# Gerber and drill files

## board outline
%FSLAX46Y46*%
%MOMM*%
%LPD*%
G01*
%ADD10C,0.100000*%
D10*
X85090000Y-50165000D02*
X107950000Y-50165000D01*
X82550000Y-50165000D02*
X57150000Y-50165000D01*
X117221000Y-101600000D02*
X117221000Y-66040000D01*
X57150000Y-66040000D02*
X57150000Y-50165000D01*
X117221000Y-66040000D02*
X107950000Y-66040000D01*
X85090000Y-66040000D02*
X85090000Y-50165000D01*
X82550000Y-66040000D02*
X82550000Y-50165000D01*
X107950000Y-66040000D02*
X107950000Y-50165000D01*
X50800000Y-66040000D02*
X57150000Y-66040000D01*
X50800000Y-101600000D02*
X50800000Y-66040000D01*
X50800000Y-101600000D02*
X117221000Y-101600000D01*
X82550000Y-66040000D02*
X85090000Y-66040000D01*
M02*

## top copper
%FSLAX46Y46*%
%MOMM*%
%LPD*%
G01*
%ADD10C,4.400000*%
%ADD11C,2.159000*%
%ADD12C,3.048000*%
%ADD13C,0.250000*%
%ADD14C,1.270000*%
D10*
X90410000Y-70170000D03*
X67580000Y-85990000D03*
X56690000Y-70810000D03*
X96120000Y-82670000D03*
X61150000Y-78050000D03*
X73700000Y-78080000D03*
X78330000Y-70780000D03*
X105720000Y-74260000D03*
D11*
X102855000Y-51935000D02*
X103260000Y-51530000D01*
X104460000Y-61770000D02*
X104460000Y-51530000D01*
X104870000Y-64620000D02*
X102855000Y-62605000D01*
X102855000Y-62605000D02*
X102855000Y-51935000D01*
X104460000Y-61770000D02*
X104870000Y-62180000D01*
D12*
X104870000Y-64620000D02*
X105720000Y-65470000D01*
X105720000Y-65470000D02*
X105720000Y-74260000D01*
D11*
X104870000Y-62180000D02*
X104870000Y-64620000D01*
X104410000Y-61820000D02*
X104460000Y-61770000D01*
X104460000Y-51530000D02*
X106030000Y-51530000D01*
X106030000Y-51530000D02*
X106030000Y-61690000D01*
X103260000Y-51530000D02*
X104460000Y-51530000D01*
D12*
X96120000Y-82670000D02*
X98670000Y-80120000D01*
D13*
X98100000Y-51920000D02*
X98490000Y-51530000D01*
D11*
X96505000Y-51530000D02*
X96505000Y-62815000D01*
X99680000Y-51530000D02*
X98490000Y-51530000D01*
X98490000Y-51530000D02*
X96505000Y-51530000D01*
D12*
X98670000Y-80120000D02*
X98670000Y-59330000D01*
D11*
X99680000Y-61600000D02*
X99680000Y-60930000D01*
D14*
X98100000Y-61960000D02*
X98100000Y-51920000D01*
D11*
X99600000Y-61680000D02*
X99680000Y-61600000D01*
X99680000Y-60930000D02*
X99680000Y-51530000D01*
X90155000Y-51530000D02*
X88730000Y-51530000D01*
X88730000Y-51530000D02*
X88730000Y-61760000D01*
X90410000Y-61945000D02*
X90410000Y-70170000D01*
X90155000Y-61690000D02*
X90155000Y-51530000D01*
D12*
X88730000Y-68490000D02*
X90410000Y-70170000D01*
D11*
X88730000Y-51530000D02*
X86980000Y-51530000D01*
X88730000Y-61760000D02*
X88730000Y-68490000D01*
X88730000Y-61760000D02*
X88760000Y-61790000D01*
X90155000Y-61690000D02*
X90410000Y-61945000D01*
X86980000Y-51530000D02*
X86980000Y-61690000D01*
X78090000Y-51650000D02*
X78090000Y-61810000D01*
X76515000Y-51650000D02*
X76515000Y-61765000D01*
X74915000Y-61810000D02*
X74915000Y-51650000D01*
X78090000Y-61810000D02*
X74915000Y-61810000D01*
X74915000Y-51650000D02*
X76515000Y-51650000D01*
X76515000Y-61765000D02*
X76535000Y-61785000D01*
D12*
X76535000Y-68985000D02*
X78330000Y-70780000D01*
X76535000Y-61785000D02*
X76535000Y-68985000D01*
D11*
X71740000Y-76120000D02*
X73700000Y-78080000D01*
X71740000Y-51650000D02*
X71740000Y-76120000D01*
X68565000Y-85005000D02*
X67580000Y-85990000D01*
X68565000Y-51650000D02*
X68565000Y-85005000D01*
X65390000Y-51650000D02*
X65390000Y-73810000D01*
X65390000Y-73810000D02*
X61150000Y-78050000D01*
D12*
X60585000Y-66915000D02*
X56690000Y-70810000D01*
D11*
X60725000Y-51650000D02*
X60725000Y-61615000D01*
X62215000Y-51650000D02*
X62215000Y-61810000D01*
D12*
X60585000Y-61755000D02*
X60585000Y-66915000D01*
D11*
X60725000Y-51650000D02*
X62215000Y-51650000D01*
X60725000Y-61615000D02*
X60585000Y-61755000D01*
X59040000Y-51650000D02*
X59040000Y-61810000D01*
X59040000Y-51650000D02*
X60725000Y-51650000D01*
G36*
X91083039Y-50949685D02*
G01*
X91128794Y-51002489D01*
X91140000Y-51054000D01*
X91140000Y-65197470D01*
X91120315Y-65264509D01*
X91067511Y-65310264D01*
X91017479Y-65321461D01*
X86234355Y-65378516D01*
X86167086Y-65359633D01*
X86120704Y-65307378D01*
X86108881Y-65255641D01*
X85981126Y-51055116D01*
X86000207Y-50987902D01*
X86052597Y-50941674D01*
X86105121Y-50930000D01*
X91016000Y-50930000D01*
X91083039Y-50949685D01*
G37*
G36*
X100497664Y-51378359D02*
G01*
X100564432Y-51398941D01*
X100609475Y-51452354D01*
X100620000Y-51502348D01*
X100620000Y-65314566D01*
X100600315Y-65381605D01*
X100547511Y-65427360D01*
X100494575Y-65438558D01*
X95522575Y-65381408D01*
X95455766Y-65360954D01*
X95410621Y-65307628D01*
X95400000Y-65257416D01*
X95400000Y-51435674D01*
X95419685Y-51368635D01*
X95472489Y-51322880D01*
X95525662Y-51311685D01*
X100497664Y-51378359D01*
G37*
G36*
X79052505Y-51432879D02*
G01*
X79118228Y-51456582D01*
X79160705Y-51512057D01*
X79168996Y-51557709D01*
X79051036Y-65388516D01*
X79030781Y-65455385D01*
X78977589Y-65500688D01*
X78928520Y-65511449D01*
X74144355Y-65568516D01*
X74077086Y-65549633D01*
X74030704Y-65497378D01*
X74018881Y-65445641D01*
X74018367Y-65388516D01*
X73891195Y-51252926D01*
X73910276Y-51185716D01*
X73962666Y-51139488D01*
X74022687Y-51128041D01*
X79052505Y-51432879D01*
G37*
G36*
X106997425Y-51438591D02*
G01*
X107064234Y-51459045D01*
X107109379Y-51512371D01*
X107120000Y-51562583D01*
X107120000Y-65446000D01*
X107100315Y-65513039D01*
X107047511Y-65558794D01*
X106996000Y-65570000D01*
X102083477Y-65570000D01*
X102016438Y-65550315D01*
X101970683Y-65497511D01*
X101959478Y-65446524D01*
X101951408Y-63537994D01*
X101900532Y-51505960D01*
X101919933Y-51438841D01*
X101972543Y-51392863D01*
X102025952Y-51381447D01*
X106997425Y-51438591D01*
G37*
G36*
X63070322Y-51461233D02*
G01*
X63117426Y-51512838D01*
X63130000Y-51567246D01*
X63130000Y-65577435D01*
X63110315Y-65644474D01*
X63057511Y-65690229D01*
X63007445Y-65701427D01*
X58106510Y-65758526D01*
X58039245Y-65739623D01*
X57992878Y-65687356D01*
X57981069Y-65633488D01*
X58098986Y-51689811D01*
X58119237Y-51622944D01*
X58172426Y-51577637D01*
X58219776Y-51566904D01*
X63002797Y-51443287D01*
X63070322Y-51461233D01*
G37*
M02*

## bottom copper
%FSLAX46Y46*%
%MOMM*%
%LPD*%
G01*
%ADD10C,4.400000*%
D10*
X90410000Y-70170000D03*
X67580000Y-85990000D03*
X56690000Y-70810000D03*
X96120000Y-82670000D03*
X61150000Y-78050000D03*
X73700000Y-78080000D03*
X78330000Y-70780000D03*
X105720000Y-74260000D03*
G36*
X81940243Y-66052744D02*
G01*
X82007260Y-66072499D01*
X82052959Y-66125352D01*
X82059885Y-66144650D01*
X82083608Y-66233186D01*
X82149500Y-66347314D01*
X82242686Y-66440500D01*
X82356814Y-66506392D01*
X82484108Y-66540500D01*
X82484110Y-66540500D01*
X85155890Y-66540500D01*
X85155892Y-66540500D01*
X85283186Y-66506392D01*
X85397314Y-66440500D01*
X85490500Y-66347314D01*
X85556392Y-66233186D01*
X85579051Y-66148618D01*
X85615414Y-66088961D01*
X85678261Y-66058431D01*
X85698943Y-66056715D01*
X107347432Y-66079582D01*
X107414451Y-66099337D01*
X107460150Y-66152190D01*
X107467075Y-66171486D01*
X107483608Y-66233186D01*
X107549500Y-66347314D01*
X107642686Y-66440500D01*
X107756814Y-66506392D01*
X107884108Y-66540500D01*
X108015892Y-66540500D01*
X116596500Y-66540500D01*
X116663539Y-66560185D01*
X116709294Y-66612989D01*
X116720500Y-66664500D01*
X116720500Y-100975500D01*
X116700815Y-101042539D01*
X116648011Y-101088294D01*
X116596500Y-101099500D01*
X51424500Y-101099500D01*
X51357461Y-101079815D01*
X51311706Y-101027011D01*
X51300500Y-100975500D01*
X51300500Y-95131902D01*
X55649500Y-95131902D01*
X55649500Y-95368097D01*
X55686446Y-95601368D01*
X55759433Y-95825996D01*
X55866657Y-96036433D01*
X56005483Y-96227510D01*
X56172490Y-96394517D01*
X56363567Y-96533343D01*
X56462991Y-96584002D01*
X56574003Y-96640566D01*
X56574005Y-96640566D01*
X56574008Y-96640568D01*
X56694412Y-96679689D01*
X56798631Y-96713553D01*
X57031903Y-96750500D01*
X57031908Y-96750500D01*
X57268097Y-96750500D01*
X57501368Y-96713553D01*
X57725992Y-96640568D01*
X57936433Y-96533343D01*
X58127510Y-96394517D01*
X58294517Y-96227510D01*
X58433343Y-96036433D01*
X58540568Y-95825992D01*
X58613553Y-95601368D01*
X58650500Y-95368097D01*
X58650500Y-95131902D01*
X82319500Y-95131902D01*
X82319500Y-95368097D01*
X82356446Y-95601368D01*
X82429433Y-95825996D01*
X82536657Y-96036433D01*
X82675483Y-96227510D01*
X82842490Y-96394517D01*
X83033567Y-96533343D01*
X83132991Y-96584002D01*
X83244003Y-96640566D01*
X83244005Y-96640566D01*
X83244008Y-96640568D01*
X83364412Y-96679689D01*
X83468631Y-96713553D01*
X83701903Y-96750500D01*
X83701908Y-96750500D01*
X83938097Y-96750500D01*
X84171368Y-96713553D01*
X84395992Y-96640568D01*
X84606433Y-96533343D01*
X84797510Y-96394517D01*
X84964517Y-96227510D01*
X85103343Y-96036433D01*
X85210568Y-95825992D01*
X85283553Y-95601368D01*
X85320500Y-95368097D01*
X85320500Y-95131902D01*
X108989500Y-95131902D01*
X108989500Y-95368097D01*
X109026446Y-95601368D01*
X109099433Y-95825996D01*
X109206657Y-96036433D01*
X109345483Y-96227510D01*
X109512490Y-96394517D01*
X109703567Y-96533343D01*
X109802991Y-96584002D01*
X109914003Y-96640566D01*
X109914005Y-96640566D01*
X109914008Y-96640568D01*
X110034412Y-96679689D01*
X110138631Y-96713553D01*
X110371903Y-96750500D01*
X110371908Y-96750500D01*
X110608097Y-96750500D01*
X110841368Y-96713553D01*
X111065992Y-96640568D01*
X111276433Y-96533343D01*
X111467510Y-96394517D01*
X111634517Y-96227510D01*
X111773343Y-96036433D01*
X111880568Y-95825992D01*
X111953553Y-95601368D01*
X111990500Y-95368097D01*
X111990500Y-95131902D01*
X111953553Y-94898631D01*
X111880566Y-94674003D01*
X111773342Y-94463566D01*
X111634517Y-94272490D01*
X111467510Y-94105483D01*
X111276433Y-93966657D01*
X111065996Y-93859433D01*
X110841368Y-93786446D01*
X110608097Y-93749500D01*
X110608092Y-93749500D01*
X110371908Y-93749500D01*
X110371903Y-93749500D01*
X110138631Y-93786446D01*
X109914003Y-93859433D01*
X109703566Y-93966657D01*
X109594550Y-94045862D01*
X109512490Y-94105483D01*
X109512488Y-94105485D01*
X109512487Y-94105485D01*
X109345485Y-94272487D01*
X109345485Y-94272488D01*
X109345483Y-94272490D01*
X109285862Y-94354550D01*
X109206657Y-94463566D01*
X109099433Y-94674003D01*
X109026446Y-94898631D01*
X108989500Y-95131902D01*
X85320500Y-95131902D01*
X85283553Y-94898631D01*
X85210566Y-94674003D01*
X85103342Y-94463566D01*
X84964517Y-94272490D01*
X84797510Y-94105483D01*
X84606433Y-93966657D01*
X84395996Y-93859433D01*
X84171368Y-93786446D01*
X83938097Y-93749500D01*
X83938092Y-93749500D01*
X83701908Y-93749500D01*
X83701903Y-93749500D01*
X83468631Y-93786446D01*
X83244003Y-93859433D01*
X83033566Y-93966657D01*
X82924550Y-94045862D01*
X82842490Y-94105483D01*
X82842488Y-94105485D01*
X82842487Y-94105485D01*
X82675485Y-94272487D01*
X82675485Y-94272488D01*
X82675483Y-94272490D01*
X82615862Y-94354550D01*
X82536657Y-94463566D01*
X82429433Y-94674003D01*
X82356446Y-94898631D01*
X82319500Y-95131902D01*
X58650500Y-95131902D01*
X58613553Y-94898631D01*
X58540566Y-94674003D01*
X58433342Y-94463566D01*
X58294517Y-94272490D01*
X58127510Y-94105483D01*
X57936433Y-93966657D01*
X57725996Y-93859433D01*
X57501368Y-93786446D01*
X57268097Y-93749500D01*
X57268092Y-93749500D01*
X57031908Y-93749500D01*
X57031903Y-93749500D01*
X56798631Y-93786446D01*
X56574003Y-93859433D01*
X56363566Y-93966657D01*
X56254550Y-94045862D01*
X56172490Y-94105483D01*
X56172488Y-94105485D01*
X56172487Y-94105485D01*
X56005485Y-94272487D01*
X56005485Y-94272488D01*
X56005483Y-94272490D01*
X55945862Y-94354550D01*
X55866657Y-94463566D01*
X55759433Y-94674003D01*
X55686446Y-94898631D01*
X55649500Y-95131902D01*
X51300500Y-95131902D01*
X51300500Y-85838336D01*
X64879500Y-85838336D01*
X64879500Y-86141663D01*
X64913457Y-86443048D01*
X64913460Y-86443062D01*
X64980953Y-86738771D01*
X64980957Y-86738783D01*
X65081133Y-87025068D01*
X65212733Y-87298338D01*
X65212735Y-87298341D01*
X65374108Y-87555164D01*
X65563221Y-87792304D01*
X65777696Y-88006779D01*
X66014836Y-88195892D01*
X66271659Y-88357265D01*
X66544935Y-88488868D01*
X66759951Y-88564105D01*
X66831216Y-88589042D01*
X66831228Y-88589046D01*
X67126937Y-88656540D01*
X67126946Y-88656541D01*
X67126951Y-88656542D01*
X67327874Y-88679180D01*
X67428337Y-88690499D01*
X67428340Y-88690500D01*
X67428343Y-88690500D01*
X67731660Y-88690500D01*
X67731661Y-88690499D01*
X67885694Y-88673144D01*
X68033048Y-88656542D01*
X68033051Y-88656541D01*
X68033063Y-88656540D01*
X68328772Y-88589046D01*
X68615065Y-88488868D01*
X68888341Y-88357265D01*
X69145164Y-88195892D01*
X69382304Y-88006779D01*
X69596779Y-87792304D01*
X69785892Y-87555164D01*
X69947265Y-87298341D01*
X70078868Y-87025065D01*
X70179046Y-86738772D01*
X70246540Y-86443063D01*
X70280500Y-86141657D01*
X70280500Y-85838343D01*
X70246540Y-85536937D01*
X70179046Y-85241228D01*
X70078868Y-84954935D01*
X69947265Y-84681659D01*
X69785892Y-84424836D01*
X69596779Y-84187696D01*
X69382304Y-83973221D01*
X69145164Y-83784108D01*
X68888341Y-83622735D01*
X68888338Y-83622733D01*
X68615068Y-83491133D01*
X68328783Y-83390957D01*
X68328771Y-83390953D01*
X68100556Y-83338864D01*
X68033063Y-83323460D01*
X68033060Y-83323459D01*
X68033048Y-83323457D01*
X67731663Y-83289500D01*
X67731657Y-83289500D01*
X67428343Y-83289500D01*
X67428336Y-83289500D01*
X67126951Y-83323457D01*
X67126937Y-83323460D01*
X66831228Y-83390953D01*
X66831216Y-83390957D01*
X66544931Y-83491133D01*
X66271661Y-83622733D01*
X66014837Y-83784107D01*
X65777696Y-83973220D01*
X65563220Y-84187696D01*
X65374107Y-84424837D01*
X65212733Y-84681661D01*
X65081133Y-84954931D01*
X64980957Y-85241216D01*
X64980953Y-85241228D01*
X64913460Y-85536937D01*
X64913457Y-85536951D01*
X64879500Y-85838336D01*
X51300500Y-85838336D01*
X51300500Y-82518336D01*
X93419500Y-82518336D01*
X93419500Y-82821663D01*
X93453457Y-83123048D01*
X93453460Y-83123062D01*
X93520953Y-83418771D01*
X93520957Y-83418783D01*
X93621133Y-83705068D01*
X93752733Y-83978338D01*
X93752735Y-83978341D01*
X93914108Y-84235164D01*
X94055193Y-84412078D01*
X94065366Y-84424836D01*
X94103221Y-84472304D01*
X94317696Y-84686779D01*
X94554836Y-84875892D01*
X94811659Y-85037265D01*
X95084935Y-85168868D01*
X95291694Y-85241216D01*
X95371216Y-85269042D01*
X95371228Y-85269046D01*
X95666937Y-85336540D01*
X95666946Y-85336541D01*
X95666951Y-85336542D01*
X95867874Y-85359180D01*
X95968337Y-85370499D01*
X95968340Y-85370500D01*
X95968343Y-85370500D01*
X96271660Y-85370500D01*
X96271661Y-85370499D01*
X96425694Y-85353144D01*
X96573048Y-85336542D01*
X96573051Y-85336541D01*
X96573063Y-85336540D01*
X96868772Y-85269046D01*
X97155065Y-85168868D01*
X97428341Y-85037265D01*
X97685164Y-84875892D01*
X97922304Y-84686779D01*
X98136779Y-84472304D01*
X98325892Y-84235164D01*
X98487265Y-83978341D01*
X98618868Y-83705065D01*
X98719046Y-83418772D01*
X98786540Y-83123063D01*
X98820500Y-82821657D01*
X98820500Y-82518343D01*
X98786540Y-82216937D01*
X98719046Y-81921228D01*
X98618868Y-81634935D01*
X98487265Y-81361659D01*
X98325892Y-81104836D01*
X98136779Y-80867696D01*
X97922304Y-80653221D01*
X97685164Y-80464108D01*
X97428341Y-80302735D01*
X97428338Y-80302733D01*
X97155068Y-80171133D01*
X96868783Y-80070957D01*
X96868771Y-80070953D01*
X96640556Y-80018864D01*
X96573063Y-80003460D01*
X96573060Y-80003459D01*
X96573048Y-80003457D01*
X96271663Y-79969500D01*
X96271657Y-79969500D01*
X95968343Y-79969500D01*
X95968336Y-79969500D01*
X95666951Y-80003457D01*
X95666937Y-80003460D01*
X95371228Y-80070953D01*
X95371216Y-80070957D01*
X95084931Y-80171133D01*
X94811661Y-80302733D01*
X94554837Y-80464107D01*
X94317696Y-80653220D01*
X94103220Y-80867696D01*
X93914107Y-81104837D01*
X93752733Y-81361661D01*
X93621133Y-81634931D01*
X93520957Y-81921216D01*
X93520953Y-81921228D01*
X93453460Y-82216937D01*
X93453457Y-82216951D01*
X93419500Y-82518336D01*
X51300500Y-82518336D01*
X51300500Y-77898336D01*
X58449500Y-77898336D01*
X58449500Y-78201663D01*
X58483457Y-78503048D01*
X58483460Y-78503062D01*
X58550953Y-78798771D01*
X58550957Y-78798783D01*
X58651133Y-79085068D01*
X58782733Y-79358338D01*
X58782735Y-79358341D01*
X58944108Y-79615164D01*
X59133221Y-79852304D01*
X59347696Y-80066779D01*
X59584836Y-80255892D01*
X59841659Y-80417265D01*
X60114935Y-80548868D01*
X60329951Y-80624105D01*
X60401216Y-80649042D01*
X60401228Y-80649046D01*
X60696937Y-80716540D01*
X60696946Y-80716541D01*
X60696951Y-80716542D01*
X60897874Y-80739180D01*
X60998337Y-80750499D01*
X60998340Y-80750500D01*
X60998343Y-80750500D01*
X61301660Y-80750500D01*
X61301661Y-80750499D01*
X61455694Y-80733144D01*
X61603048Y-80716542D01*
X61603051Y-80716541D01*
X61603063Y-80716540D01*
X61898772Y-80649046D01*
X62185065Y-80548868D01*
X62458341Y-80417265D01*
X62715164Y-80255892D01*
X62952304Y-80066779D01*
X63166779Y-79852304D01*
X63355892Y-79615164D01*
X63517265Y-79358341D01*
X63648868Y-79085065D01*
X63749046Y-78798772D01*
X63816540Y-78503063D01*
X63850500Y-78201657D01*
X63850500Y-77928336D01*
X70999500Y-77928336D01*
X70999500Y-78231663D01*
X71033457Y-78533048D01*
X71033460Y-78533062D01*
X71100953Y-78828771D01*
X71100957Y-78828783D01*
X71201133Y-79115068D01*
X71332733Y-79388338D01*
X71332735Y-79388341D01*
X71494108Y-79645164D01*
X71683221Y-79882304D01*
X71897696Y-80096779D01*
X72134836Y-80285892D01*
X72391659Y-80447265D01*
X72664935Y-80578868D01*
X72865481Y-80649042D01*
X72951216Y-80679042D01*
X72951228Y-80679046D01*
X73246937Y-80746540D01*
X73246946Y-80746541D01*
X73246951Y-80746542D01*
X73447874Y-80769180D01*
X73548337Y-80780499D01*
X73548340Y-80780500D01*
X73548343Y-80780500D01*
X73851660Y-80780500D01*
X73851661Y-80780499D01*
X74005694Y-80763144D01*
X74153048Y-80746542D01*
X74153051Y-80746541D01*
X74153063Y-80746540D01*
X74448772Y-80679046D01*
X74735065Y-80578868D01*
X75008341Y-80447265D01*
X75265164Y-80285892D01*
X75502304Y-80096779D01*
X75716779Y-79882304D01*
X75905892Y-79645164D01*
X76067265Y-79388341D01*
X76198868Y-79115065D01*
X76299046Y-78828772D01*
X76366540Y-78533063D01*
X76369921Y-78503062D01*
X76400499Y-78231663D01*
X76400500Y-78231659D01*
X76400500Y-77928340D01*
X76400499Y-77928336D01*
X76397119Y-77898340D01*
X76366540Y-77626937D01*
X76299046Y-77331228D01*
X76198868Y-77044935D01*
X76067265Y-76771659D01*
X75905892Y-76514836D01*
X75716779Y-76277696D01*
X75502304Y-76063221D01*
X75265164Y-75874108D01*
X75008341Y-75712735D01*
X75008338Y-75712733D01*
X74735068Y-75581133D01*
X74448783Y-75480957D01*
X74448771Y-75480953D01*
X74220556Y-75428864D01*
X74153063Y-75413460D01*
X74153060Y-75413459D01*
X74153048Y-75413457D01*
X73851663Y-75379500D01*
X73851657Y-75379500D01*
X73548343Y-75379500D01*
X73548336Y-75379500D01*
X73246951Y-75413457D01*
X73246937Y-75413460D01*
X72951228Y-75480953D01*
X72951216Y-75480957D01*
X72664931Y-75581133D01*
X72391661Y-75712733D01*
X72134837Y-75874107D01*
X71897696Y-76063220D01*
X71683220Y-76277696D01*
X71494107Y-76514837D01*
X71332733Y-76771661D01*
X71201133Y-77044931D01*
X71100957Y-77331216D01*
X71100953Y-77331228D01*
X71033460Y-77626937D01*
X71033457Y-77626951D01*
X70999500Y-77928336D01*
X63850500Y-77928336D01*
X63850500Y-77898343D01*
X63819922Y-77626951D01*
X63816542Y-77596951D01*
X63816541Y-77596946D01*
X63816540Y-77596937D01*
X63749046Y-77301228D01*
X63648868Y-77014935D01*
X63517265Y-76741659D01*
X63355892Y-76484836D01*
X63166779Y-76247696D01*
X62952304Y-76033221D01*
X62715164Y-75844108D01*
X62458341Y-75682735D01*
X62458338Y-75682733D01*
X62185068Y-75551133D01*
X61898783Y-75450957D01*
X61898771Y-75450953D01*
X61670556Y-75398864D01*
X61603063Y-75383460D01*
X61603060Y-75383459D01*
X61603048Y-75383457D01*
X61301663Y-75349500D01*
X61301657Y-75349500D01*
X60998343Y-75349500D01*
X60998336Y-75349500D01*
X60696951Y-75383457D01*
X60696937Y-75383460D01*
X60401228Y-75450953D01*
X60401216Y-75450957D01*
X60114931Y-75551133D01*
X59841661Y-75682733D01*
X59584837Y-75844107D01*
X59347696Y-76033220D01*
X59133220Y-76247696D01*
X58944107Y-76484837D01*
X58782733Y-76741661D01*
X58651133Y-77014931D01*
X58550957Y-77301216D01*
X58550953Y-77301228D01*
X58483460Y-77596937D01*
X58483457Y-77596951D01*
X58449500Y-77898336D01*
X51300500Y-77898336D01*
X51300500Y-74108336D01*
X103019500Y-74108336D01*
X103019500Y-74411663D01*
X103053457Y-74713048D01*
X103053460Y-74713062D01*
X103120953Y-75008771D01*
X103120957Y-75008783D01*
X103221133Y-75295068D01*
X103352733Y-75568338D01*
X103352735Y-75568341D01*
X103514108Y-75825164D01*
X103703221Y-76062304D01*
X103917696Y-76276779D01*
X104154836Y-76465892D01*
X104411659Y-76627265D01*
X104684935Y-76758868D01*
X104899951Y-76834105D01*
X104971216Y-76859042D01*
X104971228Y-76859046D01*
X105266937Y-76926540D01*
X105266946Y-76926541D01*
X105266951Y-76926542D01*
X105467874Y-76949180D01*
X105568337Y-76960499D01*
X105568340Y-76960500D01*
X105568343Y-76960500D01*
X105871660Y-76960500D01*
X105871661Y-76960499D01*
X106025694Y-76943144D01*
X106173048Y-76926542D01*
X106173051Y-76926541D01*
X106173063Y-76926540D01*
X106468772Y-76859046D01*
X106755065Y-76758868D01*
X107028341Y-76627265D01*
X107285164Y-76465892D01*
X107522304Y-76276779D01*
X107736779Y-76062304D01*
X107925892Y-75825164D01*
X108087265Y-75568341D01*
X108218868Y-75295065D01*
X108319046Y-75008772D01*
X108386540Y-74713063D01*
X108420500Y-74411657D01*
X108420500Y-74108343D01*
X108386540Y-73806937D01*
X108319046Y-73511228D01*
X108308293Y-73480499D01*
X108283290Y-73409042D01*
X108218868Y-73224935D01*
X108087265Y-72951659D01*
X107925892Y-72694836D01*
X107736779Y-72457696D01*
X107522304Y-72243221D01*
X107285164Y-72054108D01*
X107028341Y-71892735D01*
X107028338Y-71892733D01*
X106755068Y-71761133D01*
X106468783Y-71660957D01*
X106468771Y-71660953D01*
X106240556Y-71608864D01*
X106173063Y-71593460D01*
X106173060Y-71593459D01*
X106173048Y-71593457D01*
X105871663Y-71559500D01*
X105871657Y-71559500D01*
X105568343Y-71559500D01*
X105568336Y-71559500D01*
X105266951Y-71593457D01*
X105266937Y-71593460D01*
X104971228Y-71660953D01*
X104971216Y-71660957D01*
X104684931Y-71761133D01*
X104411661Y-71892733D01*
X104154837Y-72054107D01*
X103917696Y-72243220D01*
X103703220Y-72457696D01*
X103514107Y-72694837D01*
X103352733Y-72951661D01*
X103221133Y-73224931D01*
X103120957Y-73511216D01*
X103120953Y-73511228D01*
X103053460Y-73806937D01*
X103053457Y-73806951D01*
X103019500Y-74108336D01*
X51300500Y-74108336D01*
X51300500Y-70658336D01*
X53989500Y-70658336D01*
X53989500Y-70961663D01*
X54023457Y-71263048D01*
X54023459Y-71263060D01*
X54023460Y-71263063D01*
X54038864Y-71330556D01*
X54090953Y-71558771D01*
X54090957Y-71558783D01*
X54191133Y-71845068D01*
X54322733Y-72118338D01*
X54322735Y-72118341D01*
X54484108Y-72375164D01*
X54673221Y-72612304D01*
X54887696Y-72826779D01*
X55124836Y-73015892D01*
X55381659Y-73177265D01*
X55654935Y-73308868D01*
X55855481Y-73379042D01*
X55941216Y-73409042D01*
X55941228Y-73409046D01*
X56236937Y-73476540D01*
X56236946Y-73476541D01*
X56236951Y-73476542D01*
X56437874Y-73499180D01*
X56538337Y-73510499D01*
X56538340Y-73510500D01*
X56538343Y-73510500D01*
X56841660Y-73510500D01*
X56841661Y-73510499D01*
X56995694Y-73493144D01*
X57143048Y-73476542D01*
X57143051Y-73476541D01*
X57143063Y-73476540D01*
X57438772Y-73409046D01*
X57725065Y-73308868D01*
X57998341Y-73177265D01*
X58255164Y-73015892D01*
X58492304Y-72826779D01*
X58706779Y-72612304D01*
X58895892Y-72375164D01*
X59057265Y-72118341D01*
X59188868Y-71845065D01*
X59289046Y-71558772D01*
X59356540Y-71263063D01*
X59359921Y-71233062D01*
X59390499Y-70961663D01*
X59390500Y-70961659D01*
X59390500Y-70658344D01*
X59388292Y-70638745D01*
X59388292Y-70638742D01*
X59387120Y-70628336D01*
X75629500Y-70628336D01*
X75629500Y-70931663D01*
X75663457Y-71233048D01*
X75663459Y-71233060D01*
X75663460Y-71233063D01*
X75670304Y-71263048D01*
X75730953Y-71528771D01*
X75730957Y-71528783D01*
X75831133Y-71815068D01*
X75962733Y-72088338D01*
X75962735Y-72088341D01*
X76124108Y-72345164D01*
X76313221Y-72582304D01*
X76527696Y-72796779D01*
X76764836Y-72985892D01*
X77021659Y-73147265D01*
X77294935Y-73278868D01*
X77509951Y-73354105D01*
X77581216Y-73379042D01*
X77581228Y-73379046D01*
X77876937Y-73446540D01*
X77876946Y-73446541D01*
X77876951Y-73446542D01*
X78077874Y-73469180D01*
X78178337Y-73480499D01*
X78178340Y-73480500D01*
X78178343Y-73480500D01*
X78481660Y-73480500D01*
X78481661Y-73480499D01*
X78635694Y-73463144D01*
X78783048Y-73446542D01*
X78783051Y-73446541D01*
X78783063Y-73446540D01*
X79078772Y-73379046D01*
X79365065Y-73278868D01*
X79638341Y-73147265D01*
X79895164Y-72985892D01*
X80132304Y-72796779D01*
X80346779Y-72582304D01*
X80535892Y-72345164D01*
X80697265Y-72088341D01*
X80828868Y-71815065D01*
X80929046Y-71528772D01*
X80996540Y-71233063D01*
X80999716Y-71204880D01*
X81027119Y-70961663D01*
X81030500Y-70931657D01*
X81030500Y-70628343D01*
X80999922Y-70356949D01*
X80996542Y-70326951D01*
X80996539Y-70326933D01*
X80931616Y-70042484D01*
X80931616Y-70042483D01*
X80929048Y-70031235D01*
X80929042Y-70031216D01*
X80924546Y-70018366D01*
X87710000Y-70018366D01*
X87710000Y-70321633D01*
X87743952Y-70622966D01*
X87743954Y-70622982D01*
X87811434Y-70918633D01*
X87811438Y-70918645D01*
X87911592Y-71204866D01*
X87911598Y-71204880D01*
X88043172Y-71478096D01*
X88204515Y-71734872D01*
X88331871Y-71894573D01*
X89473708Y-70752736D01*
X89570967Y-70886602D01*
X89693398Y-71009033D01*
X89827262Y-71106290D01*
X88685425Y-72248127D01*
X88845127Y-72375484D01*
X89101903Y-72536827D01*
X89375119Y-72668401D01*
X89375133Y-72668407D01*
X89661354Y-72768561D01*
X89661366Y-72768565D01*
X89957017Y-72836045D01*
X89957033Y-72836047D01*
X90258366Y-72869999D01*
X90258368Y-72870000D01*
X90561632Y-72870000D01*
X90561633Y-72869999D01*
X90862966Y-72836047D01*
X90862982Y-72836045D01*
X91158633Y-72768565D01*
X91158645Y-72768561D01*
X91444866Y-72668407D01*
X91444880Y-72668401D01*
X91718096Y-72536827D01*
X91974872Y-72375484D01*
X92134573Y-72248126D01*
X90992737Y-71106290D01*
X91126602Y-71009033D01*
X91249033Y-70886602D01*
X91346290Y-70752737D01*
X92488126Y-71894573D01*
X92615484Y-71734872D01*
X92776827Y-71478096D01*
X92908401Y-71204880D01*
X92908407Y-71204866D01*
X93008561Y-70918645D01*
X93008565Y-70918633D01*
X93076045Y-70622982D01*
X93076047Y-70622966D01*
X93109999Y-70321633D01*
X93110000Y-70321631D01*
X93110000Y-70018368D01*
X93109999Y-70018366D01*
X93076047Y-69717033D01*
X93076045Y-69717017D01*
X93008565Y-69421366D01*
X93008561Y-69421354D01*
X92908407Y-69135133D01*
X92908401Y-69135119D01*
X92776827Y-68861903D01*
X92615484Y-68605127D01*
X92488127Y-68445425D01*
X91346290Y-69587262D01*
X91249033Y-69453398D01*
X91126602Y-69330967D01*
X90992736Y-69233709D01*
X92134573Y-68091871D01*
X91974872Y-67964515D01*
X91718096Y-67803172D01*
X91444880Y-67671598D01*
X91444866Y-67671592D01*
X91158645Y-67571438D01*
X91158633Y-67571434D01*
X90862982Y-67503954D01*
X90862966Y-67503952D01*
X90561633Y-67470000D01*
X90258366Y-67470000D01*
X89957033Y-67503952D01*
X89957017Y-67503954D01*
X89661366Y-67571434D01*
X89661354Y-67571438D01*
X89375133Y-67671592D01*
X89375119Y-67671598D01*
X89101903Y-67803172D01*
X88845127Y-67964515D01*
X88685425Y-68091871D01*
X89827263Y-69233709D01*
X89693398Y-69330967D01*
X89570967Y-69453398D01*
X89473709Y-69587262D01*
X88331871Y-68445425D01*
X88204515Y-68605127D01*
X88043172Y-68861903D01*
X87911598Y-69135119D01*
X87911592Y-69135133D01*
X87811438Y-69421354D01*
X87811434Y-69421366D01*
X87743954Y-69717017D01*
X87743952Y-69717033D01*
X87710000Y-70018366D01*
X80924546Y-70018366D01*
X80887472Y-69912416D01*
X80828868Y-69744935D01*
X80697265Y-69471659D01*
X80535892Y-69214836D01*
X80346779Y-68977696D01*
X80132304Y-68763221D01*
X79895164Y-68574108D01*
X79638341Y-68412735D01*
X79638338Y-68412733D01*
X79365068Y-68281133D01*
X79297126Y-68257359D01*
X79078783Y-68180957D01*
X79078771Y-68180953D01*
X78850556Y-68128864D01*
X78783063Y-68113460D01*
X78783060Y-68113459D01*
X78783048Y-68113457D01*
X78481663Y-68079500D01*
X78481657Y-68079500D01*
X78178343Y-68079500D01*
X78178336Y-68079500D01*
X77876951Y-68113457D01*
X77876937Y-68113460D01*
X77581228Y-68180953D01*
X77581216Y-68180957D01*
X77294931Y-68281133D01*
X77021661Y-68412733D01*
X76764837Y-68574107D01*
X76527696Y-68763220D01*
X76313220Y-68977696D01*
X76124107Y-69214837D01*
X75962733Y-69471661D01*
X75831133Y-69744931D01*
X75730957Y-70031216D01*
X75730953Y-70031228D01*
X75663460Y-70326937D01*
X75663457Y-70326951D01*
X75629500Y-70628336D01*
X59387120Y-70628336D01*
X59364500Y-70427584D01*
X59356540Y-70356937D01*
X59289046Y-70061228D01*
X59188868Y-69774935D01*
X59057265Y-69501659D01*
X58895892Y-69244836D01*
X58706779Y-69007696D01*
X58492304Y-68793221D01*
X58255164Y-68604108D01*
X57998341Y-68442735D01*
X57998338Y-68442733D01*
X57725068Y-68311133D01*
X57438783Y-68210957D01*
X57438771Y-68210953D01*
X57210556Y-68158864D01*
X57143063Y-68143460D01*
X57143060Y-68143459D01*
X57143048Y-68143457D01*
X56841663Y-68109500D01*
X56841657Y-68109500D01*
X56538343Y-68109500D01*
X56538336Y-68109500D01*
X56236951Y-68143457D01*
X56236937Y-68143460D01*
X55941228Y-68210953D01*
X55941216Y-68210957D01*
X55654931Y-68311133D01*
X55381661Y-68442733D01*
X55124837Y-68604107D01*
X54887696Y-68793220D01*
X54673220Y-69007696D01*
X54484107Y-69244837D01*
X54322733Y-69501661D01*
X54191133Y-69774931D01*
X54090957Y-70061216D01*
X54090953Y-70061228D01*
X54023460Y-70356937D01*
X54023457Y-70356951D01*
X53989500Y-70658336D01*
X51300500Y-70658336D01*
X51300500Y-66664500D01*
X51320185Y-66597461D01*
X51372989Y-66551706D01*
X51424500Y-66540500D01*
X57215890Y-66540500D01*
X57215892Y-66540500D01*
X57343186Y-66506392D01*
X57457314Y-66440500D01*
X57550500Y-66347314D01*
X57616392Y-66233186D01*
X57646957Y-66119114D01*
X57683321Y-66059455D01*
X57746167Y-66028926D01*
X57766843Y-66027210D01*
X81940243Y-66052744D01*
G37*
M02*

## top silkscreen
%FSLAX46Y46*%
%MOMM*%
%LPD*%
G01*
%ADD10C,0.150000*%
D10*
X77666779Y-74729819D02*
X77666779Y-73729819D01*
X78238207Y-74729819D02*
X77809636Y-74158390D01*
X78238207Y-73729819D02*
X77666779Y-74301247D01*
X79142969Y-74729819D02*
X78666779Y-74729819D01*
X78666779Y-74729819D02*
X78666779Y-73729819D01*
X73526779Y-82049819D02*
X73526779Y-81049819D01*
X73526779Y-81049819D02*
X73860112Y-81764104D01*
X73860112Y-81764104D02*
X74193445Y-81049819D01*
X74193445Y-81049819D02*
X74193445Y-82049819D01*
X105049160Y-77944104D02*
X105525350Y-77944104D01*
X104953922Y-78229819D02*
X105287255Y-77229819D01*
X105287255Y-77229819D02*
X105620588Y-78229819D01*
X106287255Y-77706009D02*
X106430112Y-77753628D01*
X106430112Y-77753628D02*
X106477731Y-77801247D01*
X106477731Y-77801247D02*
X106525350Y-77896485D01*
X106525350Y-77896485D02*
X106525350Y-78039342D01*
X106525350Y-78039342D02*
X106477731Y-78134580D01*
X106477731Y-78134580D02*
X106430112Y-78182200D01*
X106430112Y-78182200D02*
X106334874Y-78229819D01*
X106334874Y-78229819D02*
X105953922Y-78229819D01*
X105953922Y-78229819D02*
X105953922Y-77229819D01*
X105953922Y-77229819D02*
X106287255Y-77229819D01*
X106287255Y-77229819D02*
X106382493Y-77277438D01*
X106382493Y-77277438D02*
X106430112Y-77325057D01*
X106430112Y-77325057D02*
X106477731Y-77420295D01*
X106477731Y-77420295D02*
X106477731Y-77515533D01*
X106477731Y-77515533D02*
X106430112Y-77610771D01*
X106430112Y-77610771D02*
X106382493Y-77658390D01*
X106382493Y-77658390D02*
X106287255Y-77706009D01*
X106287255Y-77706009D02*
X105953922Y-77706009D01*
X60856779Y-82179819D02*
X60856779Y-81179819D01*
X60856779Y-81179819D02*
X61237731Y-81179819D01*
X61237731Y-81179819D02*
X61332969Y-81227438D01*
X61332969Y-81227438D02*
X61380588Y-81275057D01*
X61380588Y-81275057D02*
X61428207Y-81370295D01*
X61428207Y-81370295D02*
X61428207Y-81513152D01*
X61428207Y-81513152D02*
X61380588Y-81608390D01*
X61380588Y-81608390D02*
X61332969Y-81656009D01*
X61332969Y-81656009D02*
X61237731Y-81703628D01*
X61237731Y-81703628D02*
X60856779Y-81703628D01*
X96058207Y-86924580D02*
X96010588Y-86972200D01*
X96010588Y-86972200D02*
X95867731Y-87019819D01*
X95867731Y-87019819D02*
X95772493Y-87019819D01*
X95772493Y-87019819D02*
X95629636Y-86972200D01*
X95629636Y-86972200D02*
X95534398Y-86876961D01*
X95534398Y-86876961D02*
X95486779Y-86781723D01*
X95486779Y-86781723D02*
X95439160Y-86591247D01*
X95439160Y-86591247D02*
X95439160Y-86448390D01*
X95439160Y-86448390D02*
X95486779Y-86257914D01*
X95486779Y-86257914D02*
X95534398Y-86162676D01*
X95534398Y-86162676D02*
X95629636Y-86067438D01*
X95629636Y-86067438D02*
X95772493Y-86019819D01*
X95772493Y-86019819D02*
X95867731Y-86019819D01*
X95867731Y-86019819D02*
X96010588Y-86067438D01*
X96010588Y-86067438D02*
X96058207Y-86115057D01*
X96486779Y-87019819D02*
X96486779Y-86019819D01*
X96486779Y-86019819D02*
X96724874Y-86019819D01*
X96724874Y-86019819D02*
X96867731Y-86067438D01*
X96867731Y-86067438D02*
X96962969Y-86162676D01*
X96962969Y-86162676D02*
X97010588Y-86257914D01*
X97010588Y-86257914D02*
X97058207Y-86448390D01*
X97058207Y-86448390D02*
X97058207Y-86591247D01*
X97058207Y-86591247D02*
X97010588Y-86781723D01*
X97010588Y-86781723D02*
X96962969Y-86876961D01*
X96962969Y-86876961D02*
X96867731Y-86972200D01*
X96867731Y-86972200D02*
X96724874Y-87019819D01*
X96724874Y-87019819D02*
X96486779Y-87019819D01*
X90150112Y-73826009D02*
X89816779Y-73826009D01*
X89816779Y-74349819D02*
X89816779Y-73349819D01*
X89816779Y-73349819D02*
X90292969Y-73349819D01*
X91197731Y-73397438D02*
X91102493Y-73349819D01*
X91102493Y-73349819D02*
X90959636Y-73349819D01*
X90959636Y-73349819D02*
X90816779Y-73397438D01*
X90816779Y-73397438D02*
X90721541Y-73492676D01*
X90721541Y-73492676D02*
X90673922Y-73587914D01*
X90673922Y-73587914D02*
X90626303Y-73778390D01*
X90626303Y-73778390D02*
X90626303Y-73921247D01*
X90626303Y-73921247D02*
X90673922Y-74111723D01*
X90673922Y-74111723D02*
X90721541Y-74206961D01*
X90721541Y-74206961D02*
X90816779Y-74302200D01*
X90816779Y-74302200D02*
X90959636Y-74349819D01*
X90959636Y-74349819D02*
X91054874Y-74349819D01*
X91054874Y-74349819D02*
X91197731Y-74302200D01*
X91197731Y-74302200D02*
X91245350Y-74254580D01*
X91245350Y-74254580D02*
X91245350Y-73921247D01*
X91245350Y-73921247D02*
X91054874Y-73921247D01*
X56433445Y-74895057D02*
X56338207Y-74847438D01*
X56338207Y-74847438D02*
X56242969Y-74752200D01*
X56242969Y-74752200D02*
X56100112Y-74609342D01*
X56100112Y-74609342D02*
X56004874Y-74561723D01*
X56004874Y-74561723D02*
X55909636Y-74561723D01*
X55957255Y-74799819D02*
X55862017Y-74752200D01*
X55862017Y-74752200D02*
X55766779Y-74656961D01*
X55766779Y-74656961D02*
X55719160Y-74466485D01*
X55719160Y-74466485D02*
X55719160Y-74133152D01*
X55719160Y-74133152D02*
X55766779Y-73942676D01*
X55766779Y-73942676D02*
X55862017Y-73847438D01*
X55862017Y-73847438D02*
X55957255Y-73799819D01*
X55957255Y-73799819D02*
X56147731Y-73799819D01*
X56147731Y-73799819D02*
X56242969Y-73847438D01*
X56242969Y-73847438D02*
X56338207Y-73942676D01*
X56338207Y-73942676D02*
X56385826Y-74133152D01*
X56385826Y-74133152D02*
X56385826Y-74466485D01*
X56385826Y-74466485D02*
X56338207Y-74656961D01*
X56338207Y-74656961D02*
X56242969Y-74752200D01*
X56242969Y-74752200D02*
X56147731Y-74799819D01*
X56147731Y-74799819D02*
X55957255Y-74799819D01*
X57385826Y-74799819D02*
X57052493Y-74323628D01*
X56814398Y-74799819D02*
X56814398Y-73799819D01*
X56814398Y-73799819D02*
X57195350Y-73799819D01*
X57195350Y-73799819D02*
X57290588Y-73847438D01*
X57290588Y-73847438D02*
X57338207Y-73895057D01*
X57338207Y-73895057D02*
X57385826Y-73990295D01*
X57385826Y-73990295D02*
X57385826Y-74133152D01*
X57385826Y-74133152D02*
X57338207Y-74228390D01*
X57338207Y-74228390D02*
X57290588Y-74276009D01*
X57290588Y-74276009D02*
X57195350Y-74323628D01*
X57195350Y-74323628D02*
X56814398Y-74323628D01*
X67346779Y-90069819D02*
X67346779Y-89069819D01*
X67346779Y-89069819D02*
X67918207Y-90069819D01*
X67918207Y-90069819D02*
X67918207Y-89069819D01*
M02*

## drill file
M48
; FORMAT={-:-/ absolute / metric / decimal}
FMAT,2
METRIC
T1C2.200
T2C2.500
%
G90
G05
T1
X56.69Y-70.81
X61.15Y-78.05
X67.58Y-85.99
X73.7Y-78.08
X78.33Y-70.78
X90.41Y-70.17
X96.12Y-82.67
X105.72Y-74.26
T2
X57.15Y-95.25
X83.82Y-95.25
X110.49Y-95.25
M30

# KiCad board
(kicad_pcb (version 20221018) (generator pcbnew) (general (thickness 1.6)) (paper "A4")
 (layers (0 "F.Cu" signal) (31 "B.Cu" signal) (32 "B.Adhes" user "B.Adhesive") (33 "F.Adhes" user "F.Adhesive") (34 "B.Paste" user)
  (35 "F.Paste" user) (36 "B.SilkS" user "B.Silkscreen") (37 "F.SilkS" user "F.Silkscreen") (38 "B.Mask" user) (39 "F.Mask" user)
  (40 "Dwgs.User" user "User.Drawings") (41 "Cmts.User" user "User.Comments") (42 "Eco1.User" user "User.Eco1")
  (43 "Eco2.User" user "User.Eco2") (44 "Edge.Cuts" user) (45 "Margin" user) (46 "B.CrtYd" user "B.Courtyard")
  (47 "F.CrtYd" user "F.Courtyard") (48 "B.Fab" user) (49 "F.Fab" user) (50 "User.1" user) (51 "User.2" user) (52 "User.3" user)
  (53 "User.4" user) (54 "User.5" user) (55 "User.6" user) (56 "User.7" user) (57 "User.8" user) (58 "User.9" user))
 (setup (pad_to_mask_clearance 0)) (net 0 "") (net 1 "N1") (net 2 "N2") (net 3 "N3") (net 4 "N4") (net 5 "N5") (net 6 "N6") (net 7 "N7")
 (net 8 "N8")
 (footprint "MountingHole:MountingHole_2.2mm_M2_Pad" (layer "F.Cu") (at 90.41 70.17)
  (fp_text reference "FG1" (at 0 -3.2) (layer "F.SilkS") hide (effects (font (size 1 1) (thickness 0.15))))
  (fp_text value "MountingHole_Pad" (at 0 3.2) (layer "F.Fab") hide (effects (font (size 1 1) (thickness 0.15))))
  (pad "1" thru_hole circle (at 0 0) (size 4.4 4.4) (drill 2.2) (layers "*.Cu" "*.Mask") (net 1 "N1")))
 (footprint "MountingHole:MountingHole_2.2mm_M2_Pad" (layer "F.Cu") (at 67.58 85.99)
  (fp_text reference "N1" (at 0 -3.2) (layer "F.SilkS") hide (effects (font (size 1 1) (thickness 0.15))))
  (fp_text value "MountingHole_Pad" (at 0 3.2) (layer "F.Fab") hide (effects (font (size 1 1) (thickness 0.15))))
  (pad "1" thru_hole circle (at 0 0) (size 4.4 4.4) (drill 2.2) (layers "*.Cu" "*.Mask") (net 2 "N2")))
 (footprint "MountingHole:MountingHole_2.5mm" (layer "F.Cu") (at 110.49 95.25)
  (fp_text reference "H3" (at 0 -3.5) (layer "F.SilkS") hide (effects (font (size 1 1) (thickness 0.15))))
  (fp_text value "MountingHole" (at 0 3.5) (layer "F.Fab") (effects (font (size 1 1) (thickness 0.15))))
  (pad "" np_thru_hole circle (at 0 0) (size 2.5 2.5) (drill 2.5) (layers "*.Cu" "*.Mask")))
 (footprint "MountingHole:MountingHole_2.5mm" (layer "F.Cu") (at 83.82 95.25)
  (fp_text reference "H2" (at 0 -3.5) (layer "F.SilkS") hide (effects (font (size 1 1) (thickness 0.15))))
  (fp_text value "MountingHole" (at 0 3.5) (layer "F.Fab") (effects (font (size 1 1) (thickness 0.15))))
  (pad "" np_thru_hole circle (at 0 0) (size 2.5 2.5) (drill 2.5) (layers "*.Cu" "*.Mask")))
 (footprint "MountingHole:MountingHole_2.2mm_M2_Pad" (layer "F.Cu") (at 56.69 70.81)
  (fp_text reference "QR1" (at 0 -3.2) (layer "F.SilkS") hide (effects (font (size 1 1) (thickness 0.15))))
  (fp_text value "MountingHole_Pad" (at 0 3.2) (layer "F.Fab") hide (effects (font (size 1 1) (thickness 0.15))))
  (pad "1" thru_hole circle (at 0 0) (size 4.4 4.4) (drill 2.2) (layers "*.Cu" "*.Mask") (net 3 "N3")))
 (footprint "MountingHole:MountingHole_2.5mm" (layer "F.Cu") (at 57.15 95.25)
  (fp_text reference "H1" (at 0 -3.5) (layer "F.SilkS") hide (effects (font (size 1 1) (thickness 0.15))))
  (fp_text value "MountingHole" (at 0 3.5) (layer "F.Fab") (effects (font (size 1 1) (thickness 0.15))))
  (pad "" np_thru_hole circle (at 0 0) (size 2.5 2.5) (drill 2.5) (layers "*.Cu" "*.Mask")))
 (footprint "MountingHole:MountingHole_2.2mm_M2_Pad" (layer "F.Cu") (at 96.12 82.67)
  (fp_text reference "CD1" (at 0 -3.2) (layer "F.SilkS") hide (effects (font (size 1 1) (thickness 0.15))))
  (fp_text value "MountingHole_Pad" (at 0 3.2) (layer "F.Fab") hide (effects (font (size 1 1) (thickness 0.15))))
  (pad "1" thru_hole circle (at 0 0) (size 4.4 4.4) (drill 2.2) (layers "*.Cu" "*.Mask") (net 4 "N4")))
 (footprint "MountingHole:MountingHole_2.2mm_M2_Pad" (layer "F.Cu") (at 61.15 78.05)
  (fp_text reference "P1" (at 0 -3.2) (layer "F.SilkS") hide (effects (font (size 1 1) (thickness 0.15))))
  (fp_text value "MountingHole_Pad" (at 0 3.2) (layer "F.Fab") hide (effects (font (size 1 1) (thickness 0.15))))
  (pad "1" thru_hole circle (at 0 0) (size 4.4 4.4) (drill 2.2) (layers "*.Cu" "*.Mask") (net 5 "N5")))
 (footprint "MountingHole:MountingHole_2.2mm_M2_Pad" (layer "F.Cu") (at 73.7 78.08)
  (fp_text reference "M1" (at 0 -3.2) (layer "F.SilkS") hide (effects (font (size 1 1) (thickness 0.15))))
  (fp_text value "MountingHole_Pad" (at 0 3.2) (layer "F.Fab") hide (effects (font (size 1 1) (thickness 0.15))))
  (pad "1" thru_hole circle (at 0 0) (size 4.4 4.4) (drill 2.2) (layers "*.Cu" "*.Mask") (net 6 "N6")))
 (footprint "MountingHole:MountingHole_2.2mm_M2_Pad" (layer "F.Cu") (at 78.33 70.78)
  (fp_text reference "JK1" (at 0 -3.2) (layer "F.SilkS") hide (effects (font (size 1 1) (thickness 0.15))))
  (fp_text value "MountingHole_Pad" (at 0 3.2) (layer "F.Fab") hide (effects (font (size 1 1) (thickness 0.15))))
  (pad "1" thru_hole circle (at 0 0) (size 4.4 4.4) (drill 2.2) (layers "*.Cu" "*.Mask") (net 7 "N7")))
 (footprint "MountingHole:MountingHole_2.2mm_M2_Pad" (layer "F.Cu") (at 105.72 74.26)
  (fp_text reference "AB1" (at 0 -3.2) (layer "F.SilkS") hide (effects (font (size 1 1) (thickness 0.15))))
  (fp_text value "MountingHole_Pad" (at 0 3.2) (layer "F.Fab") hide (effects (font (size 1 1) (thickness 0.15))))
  (pad "1" thru_hole circle (at 0 0) (size 4.4 4.4) (drill 2.2) (layers "*.Cu" "*.Mask") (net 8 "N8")))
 (gr_line (start 85.09 50.165) (end 107.95 50.165) (stroke (width 0.1) (type default)) (layer "Edge.Cuts"))
 (gr_line (start 82.55 50.165) (end 57.15 50.165) (stroke (width 0.1) (type default)) (layer "Edge.Cuts"))
 (gr_line (start 117.221 101.6) (end 117.221 66.04) (stroke (width 0.1) (type default)) (layer "Edge.Cuts"))
 (gr_line (start 57.15 66.04) (end 57.15 50.165) (stroke (width 0.1) (type default)) (layer "Edge.Cuts"))
 (gr_line (start 117.221 66.04) (end 107.95 66.04) (stroke (width 0.1) (type default)) (layer "Edge.Cuts"))
 (gr_line (start 85.09 66.04) (end 85.09 50.165) (stroke (width 0.1) (type default)) (layer "Edge.Cuts"))
 (gr_line (start 82.55 66.04) (end 82.55 50.165) (stroke (width 0.1) (type default)) (layer "Edge.Cuts"))
 (gr_line (start 107.95 66.04) (end 107.95 50.165) (stroke (width 0.1) (type default)) (layer "Edge.Cuts"))
 (gr_line (start 50.8 66.04) (end 57.15 66.04) (stroke (width 0.1) (type default)) (layer "Edge.Cuts"))
 (gr_line (start 50.8 101.6) (end 50.8 66.04) (stroke (width 0.1) (type default)) (layer "Edge.Cuts"))
 (gr_line (start 50.8 101.6) (end 117.221 101.6) (stroke (width 0.1) (type default)) (layer "Edge.Cuts"))
 (gr_line (start 82.55 66.04) (end 85.09 66.04) (stroke (width 0.1) (type default)) (layer "Edge.Cuts"))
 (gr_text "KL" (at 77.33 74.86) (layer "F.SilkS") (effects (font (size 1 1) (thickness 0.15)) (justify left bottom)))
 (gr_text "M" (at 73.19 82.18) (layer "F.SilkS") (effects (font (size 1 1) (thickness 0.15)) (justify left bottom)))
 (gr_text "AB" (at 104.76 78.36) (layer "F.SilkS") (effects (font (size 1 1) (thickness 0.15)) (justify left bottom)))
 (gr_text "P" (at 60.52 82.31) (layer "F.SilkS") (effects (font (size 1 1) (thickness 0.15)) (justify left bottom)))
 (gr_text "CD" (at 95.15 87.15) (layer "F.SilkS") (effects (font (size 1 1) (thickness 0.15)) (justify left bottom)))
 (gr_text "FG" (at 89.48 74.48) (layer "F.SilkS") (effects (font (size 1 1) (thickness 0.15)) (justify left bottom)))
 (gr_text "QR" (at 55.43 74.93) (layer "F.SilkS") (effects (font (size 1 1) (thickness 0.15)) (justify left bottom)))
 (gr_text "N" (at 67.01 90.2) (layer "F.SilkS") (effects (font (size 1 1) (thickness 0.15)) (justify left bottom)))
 (segment (start 102.855 51.935) (end 103.26 51.53) (width 2.159) (layer "F.Cu") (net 8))
 (segment (start 104.46 61.77) (end 104.46 51.53) (width 2.159) (layer "F.Cu") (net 8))
 (segment (start 104.87 64.62) (end 102.855 62.605) (width 2.159) (layer "F.Cu") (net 8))
 (segment (start 102.855 62.605) (end 102.855 51.935) (width 2.159) (layer "F.Cu") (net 8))
 (segment (start 104.46 61.77) (end 104.87 62.18) (width 2.159) (layer "F.Cu") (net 8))
 (segment (start 104.87 64.62) (end 105.72 65.47) (width 3.048) (layer "F.Cu") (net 8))
 (segment (start 105.72 65.47) (end 105.72 74.26) (width 3.048) (layer "F.Cu") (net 8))
 (segment (start 104.87 62.18) (end 104.87 64.62) (width 2.159) (layer "F.Cu") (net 8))
 (segment (start 104.41 61.82) (end 104.46 61.77) (width 2.159) (layer "F.Cu") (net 8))
 (segment (start 104.46 51.53) (end 106.03 51.53) (width 2.159) (layer "F.Cu") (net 8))
 (segment (start 106.03 51.53) (end 106.03 61.69) (width 2.159) (layer "F.Cu") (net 8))
 (segment (start 103.26 51.53) (end 104.46 51.53) (width 2.159) (layer "F.Cu") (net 8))
 (segment (start 96.12 82.67) (end 98.67 80.12) (width 3.048) (layer "F.Cu") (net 4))
 (segment (start 98.1 51.92) (end 98.49 51.53) (width 0.25) (layer "F.Cu") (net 4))
 (segment (start 96.505 51.53) (end 96.505 62.815) (width 2.159) (layer "F.Cu") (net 4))
 (segment (start 99.68 51.53) (end 98.49 51.53) (width 2.159) (layer "F.Cu") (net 4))
 (segment (start 98.49 51.53) (end 96.505 51.53) (width 2.159) (layer "F.Cu") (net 4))
 (segment (start 98.67 80.12) (end 98.67 59.33) (width 3.048) (layer "F.Cu") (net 4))
 (segment (start 99.68 61.6) (end 99.68 60.93) (width 2.159) (layer "F.Cu") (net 4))
 (segment (start 98.1 61.96) (end 98.1 51.92) (width 1.27) (layer "F.Cu") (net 4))
 (segment (start 99.6 61.68) (end 99.68 61.6) (width 2.159) (layer "F.Cu") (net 4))
 (segment (start 99.68 60.93) (end 99.68 51.53) (width 2.159) (layer "F.Cu") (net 4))
 (segment (start 90.155 51.53) (end 88.73 51.53) (width 2.159) (layer "F.Cu") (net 1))
 (segment (start 88.73 51.53) (end 88.73 61.76) (width 2.159) (layer "F.Cu") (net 1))
 (segment (start 90.41 61.945) (end 90.41 70.17) (width 2.159) (layer "F.Cu") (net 1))
 (segment (start 90.155 61.69) (end 90.155 51.53) (width 2.159) (layer "F.Cu") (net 1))
 (segment (start 88.73 68.49) (end 90.41 70.17) (width 3.048) (layer "F.Cu") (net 1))
 (segment (start 88.73 51.53) (end 86.98 51.53) (width 2.159) (layer "F.Cu") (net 1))
 (segment (start 88.73 61.76) (end 88.73 68.49) (width 2.159) (layer "F.Cu") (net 1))
 (segment (start 88.73 61.76) (end 88.76 61.79) (width 2.159) (layer "F.Cu") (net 1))
 (segment (start 90.155 61.69) (end 90.41 61.945) (width 2.159) (layer "F.Cu") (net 1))
 (segment (start 86.98 51.53) (end 86.98 61.69) (width 2.159) (layer "F.Cu") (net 1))
 (segment (start 78.09 51.65) (end 78.09 61.81) (width 2.159) (layer "F.Cu") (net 7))
 (segment (start 76.515 51.65) (end 76.515 61.765) (width 2.159) (layer "F.Cu") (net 7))
 (segment (start 74.915 61.81) (end 74.915 51.65) (width 2.159) (layer "F.Cu") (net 7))
 (segment (start 78.09 61.81) (end 74.915 61.81) (width 2.159) (layer "F.Cu") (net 7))
 (segment (start 74.915 51.65) (end 76.515 51.65) (width 2.159) (layer "F.Cu") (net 7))
 (segment (start 76.515 61.765) (end 76.535 61.785) (width 2.159) (layer "F.Cu") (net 7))
 (segment (start 76.535 68.985) (end 78.33 70.78) (width 3.048) (layer "F.Cu") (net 7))
 (segment (start 76.535 61.785) (end 76.535 68.985) (width 3.048) (layer "F.Cu") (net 7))
 (segment (start 71.74 76.12) (end 73.7 78.08) (width 2.159) (layer "F.Cu") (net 6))
 (segment (start 71.74 51.65) (end 71.74 76.12) (width 2.159) (layer "F.Cu") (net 6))
 (segment (start 68.565 85.005) (end 67.58 85.99) (width 2.159) (layer "F.Cu") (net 2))
 (segment (start 68.565 51.65) (end 68.565 85.005) (width 2.159) (layer "F.Cu") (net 2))
 (segment (start 65.39 51.65) (end 65.39 73.81) (width 2.159) (layer "F.Cu") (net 5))
 (segment (start 65.39 73.81) (end 61.15 78.05) (width 2.159) (layer "F.Cu") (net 5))
 (segment (start 60.585 66.915) (end 56.69 70.81) (width 3.048) (layer "F.Cu") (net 3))
 (segment (start 60.725 51.65) (end 60.725 61.615) (width 2.159) (layer "F.Cu") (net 3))
 (segment (start 62.215 51.65) (end 62.215 61.81) (width 2.159) (layer "F.Cu") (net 3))
 (segment (start 60.585 61.755) (end 60.585 66.915) (width 3.048) (layer "F.Cu") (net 3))
 (segment (start 60.725 51.65) (end 62.215 51.65) (width 2.159) (layer "F.Cu") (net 3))
 (segment (start 60.725 61.615) (end 60.585 61.755) (width 2.159) (layer "F.Cu") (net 3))
 (segment (start 59.04 51.65) (end 59.04 61.81) (width 2.159) (layer "F.Cu") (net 3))
 (segment (start 59.04 51.65) (end 60.725 51.65) (width 2.159) (layer "F.Cu") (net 3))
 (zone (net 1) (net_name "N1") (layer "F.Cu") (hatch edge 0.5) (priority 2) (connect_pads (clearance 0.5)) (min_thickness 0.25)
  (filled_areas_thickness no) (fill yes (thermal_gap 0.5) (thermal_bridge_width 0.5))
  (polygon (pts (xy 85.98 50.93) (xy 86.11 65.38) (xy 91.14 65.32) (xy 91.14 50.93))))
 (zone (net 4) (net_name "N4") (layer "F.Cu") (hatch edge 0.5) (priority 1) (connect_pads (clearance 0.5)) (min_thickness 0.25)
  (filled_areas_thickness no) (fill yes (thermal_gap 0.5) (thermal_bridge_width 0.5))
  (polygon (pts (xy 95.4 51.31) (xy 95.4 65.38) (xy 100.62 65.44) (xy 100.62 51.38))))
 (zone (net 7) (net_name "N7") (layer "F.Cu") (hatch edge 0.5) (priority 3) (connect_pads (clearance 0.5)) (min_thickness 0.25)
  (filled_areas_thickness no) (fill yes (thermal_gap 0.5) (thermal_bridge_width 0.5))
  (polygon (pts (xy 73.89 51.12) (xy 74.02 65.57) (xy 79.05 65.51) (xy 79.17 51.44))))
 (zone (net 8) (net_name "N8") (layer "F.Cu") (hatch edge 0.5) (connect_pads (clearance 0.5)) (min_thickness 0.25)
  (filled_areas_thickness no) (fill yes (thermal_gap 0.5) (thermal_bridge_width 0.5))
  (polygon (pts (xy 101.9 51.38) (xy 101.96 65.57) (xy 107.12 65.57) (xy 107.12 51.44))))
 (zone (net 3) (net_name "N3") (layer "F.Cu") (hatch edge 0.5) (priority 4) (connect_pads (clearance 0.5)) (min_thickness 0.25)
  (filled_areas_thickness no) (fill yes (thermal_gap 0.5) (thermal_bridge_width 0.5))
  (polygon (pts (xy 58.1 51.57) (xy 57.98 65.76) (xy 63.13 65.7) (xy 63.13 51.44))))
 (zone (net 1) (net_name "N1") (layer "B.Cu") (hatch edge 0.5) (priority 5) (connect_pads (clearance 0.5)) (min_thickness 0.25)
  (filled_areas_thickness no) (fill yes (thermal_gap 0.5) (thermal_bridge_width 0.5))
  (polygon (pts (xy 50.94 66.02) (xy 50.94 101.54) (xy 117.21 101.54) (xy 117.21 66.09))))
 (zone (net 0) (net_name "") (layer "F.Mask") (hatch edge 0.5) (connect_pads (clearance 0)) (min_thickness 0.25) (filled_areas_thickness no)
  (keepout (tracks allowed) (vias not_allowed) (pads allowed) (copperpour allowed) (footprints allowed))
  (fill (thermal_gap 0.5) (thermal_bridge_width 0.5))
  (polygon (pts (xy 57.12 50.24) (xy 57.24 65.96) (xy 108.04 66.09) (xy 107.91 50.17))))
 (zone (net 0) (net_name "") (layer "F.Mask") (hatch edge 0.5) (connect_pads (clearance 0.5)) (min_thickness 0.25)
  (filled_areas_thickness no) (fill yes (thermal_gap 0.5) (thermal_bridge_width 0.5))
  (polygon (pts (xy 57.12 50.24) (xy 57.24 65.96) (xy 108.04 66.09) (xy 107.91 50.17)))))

